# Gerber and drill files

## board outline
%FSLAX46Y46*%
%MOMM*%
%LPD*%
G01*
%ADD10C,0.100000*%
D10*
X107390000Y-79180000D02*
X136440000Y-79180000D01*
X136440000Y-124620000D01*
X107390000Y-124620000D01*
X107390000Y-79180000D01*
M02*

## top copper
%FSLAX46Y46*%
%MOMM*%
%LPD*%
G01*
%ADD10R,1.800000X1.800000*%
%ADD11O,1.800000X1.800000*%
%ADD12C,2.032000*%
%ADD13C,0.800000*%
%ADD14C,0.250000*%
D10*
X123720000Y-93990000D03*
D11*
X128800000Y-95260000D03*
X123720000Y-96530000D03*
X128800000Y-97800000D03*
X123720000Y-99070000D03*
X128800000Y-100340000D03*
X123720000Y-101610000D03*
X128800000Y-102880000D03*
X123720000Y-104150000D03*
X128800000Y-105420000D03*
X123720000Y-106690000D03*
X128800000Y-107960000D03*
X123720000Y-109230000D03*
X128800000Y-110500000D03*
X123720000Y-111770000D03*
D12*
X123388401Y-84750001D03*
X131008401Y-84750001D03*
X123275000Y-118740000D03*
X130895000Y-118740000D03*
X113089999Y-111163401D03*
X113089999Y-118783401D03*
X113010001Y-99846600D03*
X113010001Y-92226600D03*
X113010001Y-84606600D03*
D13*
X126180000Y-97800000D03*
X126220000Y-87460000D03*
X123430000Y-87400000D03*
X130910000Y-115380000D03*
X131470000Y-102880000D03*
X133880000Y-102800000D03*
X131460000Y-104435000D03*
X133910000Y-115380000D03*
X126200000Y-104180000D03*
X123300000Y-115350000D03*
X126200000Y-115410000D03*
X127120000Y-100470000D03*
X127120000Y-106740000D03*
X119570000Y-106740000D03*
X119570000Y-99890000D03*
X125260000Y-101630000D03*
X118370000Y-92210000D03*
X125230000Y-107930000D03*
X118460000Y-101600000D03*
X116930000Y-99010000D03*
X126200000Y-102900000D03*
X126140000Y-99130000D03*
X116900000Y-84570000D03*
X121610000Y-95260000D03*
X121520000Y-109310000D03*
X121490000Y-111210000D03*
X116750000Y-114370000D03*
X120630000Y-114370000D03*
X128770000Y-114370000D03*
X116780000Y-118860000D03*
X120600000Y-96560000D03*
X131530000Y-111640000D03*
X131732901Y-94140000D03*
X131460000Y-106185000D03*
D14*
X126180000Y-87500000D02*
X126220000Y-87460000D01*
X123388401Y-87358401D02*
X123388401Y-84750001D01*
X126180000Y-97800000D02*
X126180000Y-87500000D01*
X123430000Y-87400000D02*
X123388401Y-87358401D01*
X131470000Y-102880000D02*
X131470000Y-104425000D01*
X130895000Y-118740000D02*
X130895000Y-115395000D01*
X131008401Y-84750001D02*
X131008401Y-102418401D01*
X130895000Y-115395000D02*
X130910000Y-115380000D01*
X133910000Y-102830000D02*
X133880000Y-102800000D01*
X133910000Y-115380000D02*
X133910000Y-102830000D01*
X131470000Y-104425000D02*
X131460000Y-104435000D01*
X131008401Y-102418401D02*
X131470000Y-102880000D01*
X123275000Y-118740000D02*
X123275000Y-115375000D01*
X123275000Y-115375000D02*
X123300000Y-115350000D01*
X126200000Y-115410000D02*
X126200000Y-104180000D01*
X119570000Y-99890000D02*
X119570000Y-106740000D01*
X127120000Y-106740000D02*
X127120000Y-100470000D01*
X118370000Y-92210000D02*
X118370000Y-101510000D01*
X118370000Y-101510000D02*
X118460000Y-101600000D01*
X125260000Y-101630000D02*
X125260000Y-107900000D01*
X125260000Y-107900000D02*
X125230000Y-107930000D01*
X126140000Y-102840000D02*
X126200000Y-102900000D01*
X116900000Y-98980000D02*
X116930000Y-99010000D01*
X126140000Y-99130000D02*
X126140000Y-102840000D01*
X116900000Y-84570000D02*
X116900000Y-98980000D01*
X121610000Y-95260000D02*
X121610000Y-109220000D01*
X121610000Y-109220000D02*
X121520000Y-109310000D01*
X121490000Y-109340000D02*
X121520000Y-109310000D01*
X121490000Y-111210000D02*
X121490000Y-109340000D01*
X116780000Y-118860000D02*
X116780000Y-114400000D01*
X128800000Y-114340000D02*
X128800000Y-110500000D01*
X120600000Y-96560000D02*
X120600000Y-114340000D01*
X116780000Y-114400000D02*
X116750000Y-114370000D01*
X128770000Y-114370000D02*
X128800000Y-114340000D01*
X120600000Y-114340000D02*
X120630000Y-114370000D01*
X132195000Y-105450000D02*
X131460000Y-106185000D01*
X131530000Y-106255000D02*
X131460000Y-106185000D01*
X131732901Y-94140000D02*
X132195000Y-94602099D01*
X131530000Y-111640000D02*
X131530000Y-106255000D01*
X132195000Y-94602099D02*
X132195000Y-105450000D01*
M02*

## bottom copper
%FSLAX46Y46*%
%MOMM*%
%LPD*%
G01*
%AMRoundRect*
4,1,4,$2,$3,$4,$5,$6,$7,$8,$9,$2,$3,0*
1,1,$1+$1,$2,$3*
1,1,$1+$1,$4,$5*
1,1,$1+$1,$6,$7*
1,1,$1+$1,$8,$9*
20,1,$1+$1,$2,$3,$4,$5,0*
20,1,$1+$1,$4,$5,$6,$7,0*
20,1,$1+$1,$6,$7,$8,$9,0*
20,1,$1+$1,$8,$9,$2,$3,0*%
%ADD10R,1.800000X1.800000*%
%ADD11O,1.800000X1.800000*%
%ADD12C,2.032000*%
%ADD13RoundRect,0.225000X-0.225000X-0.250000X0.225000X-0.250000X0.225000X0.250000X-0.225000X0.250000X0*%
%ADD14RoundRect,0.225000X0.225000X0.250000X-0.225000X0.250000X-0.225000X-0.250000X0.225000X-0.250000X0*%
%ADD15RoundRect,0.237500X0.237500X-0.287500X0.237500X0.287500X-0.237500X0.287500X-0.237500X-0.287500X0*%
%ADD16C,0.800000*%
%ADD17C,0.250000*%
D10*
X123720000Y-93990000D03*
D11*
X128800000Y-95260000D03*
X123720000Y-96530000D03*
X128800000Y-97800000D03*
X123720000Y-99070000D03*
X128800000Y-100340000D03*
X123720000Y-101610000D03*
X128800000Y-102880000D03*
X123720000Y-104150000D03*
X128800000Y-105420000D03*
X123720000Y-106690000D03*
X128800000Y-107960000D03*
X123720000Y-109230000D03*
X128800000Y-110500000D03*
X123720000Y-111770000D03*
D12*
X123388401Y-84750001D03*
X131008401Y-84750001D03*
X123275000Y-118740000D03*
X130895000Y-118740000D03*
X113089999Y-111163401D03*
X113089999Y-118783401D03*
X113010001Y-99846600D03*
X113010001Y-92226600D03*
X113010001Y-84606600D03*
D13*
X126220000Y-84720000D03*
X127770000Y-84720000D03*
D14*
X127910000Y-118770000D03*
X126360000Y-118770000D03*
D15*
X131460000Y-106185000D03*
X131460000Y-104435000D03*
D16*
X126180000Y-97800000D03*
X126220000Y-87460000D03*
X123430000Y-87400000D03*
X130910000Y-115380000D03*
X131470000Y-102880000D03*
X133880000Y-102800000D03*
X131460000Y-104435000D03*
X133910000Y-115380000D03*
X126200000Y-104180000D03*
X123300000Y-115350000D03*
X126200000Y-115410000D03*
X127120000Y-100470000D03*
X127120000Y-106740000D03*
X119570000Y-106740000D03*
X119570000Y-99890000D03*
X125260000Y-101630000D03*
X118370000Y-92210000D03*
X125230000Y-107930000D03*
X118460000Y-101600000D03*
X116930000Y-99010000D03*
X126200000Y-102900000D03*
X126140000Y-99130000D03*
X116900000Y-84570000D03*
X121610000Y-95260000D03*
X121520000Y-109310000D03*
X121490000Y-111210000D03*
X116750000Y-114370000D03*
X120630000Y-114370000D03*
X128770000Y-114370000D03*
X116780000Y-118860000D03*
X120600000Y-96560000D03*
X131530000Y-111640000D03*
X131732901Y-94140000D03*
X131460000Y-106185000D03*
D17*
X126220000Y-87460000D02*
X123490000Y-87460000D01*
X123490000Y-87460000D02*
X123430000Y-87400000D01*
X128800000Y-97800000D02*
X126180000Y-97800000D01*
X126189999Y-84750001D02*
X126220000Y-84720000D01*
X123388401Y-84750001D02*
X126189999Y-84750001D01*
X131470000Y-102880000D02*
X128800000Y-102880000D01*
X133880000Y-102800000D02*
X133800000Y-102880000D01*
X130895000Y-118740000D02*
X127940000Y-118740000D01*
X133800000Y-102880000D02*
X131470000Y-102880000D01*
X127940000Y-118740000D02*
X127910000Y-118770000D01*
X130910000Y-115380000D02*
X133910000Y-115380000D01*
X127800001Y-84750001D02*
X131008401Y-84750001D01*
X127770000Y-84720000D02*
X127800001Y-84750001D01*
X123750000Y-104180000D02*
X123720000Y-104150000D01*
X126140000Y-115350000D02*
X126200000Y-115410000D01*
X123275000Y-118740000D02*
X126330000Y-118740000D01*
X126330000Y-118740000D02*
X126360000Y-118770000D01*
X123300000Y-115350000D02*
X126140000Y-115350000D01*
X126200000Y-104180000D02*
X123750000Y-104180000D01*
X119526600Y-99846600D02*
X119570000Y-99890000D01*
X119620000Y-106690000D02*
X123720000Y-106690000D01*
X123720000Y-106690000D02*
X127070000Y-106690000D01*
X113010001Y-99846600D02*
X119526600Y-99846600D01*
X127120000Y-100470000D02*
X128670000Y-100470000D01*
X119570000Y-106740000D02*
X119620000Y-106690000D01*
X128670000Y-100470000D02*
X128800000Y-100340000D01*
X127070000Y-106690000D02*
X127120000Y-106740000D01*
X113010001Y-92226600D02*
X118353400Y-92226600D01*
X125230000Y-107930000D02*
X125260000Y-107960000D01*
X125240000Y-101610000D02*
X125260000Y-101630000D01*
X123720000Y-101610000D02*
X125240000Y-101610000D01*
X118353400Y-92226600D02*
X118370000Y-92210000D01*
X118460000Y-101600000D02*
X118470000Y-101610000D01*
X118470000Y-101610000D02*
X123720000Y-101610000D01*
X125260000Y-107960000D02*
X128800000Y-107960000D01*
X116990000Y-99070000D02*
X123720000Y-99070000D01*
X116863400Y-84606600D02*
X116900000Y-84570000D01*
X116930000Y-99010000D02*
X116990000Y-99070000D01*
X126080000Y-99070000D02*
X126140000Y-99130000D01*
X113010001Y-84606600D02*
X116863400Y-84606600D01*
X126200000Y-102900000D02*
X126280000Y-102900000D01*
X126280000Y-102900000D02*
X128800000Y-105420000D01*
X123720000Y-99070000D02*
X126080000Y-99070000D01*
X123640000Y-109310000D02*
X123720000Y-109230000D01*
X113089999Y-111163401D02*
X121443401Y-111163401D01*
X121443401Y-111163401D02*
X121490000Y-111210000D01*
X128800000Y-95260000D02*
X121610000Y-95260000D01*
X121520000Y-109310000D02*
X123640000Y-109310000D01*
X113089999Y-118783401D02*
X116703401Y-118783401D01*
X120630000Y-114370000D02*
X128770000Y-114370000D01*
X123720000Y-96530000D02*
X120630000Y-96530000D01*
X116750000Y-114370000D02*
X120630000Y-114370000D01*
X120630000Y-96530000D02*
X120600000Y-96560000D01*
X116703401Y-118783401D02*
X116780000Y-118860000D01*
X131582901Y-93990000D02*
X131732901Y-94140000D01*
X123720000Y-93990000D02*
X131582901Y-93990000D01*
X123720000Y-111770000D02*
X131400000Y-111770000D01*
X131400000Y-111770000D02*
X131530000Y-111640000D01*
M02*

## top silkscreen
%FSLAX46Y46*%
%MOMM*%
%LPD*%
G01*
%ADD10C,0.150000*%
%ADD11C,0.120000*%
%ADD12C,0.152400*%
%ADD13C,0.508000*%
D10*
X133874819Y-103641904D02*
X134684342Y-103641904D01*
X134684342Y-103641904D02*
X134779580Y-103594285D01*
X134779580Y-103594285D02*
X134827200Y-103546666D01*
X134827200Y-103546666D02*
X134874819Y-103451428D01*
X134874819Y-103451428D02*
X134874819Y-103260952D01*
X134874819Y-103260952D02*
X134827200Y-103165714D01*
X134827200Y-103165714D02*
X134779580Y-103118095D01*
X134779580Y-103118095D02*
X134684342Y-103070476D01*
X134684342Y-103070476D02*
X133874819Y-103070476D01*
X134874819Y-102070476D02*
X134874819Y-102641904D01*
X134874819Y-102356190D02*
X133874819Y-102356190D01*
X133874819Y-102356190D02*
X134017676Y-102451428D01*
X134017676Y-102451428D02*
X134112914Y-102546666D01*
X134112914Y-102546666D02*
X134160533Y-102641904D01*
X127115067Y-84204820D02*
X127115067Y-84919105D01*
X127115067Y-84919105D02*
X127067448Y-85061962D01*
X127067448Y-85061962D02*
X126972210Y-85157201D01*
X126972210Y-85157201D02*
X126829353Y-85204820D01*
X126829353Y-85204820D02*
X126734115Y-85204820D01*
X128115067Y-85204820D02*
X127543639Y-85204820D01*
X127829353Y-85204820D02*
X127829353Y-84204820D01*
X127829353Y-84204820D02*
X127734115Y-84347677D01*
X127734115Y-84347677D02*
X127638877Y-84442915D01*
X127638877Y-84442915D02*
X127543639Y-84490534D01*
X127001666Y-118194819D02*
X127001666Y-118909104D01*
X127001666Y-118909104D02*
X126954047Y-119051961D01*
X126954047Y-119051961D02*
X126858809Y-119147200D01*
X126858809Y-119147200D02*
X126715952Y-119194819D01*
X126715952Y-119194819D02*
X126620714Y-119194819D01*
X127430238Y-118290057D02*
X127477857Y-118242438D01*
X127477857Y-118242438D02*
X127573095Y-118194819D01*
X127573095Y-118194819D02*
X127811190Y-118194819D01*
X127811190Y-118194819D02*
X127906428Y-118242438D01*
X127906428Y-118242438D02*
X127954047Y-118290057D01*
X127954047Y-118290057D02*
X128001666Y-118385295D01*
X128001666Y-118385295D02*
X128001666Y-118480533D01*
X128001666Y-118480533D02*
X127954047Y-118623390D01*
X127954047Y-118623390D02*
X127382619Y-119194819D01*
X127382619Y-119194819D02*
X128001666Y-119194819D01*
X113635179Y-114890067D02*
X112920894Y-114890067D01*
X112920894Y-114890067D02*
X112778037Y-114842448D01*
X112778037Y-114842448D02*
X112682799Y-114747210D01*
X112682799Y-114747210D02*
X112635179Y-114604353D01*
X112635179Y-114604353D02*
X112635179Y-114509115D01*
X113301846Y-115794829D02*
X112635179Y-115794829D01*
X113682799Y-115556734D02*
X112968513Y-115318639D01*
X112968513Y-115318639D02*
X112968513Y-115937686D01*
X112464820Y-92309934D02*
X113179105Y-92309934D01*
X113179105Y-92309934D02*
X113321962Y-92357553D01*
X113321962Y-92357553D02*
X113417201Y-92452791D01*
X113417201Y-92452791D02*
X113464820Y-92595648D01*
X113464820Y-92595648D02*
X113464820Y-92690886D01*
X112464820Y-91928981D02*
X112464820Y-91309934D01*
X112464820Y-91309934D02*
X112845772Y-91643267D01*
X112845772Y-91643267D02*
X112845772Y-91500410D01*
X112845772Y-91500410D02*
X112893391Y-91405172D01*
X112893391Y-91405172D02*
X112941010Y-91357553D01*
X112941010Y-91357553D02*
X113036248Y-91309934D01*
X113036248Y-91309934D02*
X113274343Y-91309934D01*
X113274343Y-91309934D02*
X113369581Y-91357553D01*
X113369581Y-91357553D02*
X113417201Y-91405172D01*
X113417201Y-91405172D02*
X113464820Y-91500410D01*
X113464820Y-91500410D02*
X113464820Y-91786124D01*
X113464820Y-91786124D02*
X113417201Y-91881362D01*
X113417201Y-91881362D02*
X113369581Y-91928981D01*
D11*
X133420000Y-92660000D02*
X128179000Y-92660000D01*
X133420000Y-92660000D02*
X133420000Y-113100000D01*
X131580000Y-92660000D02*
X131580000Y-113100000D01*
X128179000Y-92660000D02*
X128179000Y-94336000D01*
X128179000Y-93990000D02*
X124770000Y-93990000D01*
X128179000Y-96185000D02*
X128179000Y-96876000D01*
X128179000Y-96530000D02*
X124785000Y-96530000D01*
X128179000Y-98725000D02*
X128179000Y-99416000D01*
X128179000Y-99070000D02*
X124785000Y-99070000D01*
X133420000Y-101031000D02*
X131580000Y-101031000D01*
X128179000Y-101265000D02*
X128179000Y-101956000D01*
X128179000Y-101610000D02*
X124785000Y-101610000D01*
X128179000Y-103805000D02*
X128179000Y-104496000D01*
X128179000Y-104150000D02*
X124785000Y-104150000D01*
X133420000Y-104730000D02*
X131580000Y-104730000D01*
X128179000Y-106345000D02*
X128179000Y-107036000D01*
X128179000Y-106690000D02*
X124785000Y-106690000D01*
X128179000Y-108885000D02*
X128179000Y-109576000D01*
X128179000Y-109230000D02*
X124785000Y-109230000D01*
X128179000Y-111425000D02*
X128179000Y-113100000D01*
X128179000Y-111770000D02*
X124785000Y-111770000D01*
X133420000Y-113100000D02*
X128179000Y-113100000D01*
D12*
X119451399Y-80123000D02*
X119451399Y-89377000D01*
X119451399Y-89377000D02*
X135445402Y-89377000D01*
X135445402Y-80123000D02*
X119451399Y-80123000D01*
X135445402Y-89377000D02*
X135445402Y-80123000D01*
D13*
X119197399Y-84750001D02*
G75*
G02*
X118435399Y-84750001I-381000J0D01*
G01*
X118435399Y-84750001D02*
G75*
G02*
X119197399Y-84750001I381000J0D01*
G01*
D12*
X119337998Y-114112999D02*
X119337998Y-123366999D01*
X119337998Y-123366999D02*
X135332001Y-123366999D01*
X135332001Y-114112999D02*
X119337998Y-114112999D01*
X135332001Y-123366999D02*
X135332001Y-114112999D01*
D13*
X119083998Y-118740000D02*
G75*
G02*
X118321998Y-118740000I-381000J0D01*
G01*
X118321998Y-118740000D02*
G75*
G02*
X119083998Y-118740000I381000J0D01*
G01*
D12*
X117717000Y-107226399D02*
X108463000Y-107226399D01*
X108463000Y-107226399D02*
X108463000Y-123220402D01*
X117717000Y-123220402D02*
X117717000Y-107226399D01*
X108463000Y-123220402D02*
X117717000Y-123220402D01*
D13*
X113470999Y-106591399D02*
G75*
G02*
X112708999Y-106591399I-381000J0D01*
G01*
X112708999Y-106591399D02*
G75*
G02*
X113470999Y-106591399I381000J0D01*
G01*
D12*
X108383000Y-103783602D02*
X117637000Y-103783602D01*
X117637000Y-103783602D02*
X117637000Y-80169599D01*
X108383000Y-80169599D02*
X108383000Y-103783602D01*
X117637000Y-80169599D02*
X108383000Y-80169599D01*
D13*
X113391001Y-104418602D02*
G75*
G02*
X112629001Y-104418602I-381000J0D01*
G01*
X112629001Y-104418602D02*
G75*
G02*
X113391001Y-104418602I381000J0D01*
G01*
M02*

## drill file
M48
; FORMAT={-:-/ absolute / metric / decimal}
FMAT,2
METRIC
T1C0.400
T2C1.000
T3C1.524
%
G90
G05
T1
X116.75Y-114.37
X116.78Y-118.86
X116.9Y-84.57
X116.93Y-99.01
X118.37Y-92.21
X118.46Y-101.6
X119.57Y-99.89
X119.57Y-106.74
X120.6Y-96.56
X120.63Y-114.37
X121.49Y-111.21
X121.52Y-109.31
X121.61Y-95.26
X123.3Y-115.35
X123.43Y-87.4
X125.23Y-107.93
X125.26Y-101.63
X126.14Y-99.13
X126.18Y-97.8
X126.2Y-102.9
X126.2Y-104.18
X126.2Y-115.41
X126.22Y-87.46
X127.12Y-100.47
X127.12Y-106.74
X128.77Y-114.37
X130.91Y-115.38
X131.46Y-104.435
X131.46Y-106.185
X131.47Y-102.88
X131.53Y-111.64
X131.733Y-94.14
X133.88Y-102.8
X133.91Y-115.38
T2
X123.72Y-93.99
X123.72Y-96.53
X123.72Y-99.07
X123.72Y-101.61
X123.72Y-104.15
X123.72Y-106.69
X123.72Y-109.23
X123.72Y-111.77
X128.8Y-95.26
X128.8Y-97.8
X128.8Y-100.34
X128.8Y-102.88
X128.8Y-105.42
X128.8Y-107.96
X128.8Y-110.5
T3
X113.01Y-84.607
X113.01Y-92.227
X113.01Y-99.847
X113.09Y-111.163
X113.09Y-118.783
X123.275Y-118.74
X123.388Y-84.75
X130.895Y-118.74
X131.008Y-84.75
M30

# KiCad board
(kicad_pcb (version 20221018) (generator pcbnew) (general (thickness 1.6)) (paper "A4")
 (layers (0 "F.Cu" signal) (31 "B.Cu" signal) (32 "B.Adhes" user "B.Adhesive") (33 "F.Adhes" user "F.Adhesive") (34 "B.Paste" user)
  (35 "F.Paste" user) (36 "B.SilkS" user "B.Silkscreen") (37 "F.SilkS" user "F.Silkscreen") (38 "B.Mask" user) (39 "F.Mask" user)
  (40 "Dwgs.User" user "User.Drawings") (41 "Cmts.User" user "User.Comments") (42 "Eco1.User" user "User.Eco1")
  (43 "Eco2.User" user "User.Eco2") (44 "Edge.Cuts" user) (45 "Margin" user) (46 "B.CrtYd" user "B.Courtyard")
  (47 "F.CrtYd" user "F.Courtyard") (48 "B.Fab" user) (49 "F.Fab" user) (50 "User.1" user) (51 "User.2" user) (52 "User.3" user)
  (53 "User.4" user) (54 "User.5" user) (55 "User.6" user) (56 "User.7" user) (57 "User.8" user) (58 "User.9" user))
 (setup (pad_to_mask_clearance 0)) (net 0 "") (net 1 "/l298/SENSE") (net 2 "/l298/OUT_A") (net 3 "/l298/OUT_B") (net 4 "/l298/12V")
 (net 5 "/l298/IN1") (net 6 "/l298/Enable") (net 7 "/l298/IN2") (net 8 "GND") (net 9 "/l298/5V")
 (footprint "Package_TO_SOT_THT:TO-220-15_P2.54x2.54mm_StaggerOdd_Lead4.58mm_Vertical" (layer "F.Cu") (at 123.72 93.99 -90)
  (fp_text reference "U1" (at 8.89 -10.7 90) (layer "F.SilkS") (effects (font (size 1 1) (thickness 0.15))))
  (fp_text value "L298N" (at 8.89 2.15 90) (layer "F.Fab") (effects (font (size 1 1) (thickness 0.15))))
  (fp_line (start -1.33 -9.7) (end -1.33 -4.459) (stroke (width 0.12) (type solid)) (layer "F.SilkS"))
  (fp_line (start -1.33 -9.7) (end 19.11 -9.7) (stroke (width 0.12) (type solid)) (layer "F.SilkS"))
  (fp_line (start -1.33 -7.86) (end 19.11 -7.86) (stroke (width 0.12) (type solid)) (layer "F.SilkS"))
  (fp_line (start -1.33 -4.459) (end 0.346 -4.459) (stroke (width 0.12) (type solid)) (layer "F.SilkS"))
  (fp_line (start 0 -4.459) (end 0 -1.05) (stroke (width 0.12) (type solid)) (layer "F.SilkS"))
  (fp_line (start 2.195 -4.459) (end 2.886 -4.459) (stroke (width 0.12) (type solid)) (layer "F.SilkS"))
  (fp_line (start 2.54 -4.459) (end 2.54 -1.065) (stroke (width 0.12) (type solid)) (layer "F.SilkS"))
  (fp_line (start 4.735 -4.459) (end 5.426 -4.459) (stroke (width 0.12) (type solid)) (layer "F.SilkS"))
  (fp_line (start 5.08 -4.459) (end 5.08 -1.065) (stroke (width 0.12) (type solid)) (layer "F.SilkS"))
  (fp_line (start 7.041 -9.7) (end 7.041 -7.86) (stroke (width 0.12) (type solid)) (layer "F.SilkS"))
  (fp_line (start 7.275 -4.459) (end 7.966 -4.459) (stroke (width 0.12) (type solid)) (layer "F.SilkS"))
  (fp_line (start 7.62 -4.459) (end 7.62 -1.065) (stroke (width 0.12) (type solid)) (layer "F.SilkS"))
  (fp_line (start 9.815 -4.459) (end 10.506 -4.459) (stroke (width 0.12) (type solid)) (layer "F.SilkS"))
  (fp_line (start 10.16 -4.459) (end 10.16 -1.065) (stroke (width 0.12) (type solid)) (layer "F.SilkS"))
  (fp_line (start 10.74 -9.7) (end 10.74 -7.86) (stroke (width 0.12) (type solid)) (layer "F.SilkS"))
  (fp_line (start 12.355 -4.459) (end 13.046 -4.459) (stroke (width 0.12) (type solid)) (layer "F.SilkS"))
  (fp_line (start 12.7 -4.459) (end 12.7 -1.065) (stroke (width 0.12) (type solid)) (layer "F.SilkS"))
  (fp_line (start 14.895 -4.459) (end 15.586 -4.459) (stroke (width 0.12) (type solid)) (layer "F.SilkS"))
  (fp_line (start 15.24 -4.459) (end 15.24 -1.065) (stroke (width 0.12) (type solid)) (layer "F.SilkS"))
  (fp_line (start 17.435 -4.459) (end 19.11 -4.459) (stroke (width 0.12) (type solid)) (layer "F.SilkS"))
  (fp_line (start 17.78 -4.459) (end 17.78 -1.065) (stroke (width 0.12) (type solid)) (layer "F.SilkS"))
  (fp_line (start 19.11 -9.7) (end 19.11 -4.459) (stroke (width 0.12) (type solid)) (layer "F.SilkS"))
  (pad "1" thru_hole rect (at 0 0 270) (size 1.8 1.8) (drill 1) (layers "*.Cu" "*.Mask") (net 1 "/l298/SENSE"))
  (pad "2" thru_hole oval (at 1.27 -5.08 270) (size 1.8 1.8) (drill 1) (layers "*.Cu" "*.Mask") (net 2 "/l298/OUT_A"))
  (pad "3" thru_hole oval (at 2.54 0 270) (size 1.8 1.8) (drill 1) (layers "*.Cu" "*.Mask") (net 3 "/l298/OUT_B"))
  (pad "4" thru_hole oval (at 3.81 -5.08 270) (size 1.8 1.8) (drill 1) (layers "*.Cu" "*.Mask") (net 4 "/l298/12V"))
  (pad "5" thru_hole oval (at 5.08 0 270) (size 1.8 1.8) (drill 1) (layers "*.Cu" "*.Mask") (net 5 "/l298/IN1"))
  (pad "6" thru_hole oval (at 6.35 -5.08 270) (size 1.8 1.8) (drill 1) (layers "*.Cu" "*.Mask") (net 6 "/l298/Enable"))
  (pad "7" thru_hole oval (at 7.62 0 270) (size 1.8 1.8) (drill 1) (layers "*.Cu" "*.Mask") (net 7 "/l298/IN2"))
  (pad "8" thru_hole oval (at 8.89 -5.08 270) (size 1.8 1.8) (drill 1) (layers "*.Cu" "*.Mask") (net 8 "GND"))
  (pad "9" thru_hole oval (at 10.16 0 270) (size 1.8 1.8) (drill 1) (layers "*.Cu" "*.Mask") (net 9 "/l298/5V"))
  (pad "10" thru_hole oval (at 11.43 -5.08 270) (size 1.8 1.8) (drill 1) (layers "*.Cu" "*.Mask") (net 5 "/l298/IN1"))
  (pad "11" thru_hole oval (at 12.7 0 270) (size 1.8 1.8) (drill 1) (layers "*.Cu" "*.Mask") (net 6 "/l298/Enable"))
  (pad "12" thru_hole oval (at 13.97 -5.08 270) (size 1.8 1.8) (drill 1) (layers "*.Cu" "*.Mask") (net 7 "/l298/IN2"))
  (pad "13" thru_hole oval (at 15.24 0 270) (size 1.8 1.8) (drill 1) (layers "*.Cu" "*.Mask") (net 2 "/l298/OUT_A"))
  (pad "14" thru_hole oval (at 16.51 -5.08 270) (size 1.8 1.8) (drill 1) (layers "*.Cu" "*.Mask") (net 3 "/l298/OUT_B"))
  (pad "15" thru_hole oval (at 17.78 0 270) (size 1.8 1.8) (drill 1) (layers "*.Cu" "*.Mask") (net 1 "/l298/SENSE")))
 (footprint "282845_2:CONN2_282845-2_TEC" (layer "F.Cu") (at 123.388401 84.750001)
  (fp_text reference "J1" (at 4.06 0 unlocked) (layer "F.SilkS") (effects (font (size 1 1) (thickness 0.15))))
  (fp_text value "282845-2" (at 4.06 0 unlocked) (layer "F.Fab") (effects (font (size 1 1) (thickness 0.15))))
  (fp_line (start -3.937002 -4.627001) (end -3.937002 4.626999) (stroke (width 0.1524) (type solid)) (layer "F.SilkS"))
  (fp_line (start -3.937002 4.626999) (end 12.057001 4.626999) (stroke (width 0.1524) (type solid)) (layer "F.SilkS"))
  (fp_line (start 12.057001 -4.627001) (end -3.937002 -4.627001) (stroke (width 0.1524) (type solid)) (layer "F.SilkS"))
  (fp_line (start 12.057001 4.626999) (end 12.057001 -4.627001) (stroke (width 0.1524) (type solid)) (layer "F.SilkS"))
  (fp_circle (center -4.572002 0) (end -4.191002 0) (stroke (width 0.508) (type solid)) (fill none) (layer "F.SilkS"))
  (pad "1" thru_hole circle (at 0 0) (size 2.032 2.032) (drill 1.524) (layers "*.Cu" "*.Mask") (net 4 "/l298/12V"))
  (pad "2" thru_hole circle (at 7.62 0) (size 2.032 2.032) (drill 1.524) (layers "*.Cu" "*.Mask") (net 8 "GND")))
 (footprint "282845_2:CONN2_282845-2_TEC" (layer "F.Cu") (at 123.275 118.74)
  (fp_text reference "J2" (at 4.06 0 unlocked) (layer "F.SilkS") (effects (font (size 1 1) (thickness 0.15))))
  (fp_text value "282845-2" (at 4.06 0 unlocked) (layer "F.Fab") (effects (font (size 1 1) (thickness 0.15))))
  (fp_line (start -3.937002 -4.627001) (end -3.937002 4.626999) (stroke (width 0.1524) (type solid)) (layer "F.SilkS"))
  (fp_line (start -3.937002 4.626999) (end 12.057001 4.626999) (stroke (width 0.1524) (type solid)) (layer "F.SilkS"))
  (fp_line (start 12.057001 -4.627001) (end -3.937002 -4.627001) (stroke (width 0.1524) (type solid)) (layer "F.SilkS"))
  (fp_line (start 12.057001 4.626999) (end 12.057001 -4.627001) (stroke (width 0.1524) (type solid)) (layer "F.SilkS"))
  (fp_circle (center -4.572002 0) (end -4.191002 0) (stroke (width 0.508) (type solid)) (fill none) (layer "F.SilkS"))
  (pad "1" thru_hole circle (at 0 0) (size 2.032 2.032) (drill 1.524) (layers "*.Cu" "*.Mask") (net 9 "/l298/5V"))
  (pad "2" thru_hole circle (at 7.62 0) (size 2.032 2.032) (drill 1.524) (layers "*.Cu" "*.Mask") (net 8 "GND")))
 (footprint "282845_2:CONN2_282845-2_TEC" (layer "F.Cu") (at 113.089999 111.163401 -90)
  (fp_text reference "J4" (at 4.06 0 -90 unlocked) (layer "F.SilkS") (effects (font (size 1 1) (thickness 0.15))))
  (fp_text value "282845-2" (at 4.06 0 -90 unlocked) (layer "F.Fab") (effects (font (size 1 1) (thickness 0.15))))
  (fp_line (start -3.937002 -4.627001) (end -3.937002 4.626999) (stroke (width 0.1524) (type solid)) (layer "F.SilkS"))
  (fp_line (start -3.937002 4.626999) (end 12.057001 4.626999) (stroke (width 0.1524) (type solid)) (layer "F.SilkS"))
  (fp_line (start 12.057001 -4.627001) (end -3.937002 -4.627001) (stroke (width 0.1524) (type solid)) (layer "F.SilkS"))
  (fp_line (start 12.057001 4.626999) (end 12.057001 -4.627001) (stroke (width 0.1524) (type solid)) (layer "F.SilkS"))
  (fp_circle (center -4.572002 0) (end -4.191002 0) (stroke (width 0.508) (type solid)) (fill none) (layer "F.SilkS"))
  (pad "1" thru_hole circle (at 0 0 270) (size 2.032 2.032) (drill 1.524) (layers "*.Cu" "*.Mask") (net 2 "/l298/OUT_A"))
  (pad "2" thru_hole circle (at 7.62 0 270) (size 2.032 2.032) (drill 1.524) (layers "*.Cu" "*.Mask") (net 3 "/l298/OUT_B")))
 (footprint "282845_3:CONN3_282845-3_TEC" (layer "F.Cu") (at 113.010001 99.8466 90)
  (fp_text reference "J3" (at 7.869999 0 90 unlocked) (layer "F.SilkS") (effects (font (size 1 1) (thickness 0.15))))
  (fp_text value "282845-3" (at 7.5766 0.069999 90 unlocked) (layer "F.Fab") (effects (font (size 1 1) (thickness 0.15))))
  (fp_line (start -3.937002 -4.627001) (end -3.937002 4.626999) (stroke (width 0.1524) (type solid)) (layer "F.SilkS"))
  (fp_line (start -3.937002 4.626999) (end 19.677001 4.626999) (stroke (width 0.1524) (type solid)) (layer "F.SilkS"))
  (fp_line (start 19.677001 -4.627001) (end -3.937002 -4.627001) (stroke (width 0.1524) (type solid)) (layer "F.SilkS"))
  (fp_line (start 19.677001 4.626999) (end 19.677001 -4.627001) (stroke (width 0.1524) (type solid)) (layer "F.SilkS"))
  (fp_circle (center -4.572002 0) (end -4.191002 0) (stroke (width 0.508) (type solid)) (fill none) (layer "F.SilkS"))
  (pad "1" thru_hole circle (at 0 0 90) (size 2.032 2.032) (drill 1.524) (layers "*.Cu" "*.Mask") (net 6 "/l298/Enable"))
  (pad "2" thru_hole circle (at 7.62 0 90) (size 2.032 2.032) (drill 1.524) (layers "*.Cu" "*.Mask") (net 7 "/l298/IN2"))
  (pad "3" thru_hole circle (at 15.24 0 90) (size 2.032 2.032) (drill 1.524) (layers "*.Cu" "*.Mask") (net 5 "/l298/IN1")))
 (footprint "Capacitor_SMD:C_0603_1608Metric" (layer "B.Cu") (at 126.995 84.72)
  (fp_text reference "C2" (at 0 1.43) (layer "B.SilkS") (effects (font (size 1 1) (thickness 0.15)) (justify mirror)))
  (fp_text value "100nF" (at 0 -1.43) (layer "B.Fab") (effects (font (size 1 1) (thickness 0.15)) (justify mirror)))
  (pad "1" smd roundrect (at -0.775 0) (size 0.9 0.95) (layers "B.Cu" "B.Paste" "B.Mask") (roundrect_rratio 0.25) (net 4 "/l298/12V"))
  (pad "2" smd roundrect (at 0.775 0) (size 0.9 0.95) (layers "B.Cu" "B.Paste" "B.Mask") (roundrect_rratio 0.25) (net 8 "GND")))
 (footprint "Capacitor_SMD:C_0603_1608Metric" (layer "B.Cu") (at 127.135 118.77 180)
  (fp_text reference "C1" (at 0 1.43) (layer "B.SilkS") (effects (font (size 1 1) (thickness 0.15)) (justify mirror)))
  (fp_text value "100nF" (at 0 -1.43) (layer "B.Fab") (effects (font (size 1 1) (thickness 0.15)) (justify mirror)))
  (pad "1" smd roundrect (at -0.775 0 180) (size 0.9 0.95) (layers "B.Cu" "B.Paste" "B.Mask") (roundrect_rratio 0.25) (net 8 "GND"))
  (pad "2" smd roundrect (at 0.775 0 180) (size 0.9 0.95) (layers "B.Cu" "B.Paste" "B.Mask") (roundrect_rratio 0.25) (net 9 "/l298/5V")))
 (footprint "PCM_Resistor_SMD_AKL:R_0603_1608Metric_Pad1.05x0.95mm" (layer "B.Cu") (at 131.46 105.31 90)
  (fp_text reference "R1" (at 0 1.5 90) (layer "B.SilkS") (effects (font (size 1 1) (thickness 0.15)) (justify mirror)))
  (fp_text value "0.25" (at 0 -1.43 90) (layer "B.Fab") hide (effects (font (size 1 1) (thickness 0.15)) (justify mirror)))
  (pad "1" smd roundrect (at -0.875 0 90) (size 1.05 0.95) (layers "B.Cu" "B.Paste" "B.Mask") (roundrect_rratio 0.25) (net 1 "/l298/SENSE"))
  (pad "2" smd roundrect (at 0.875 0 90) (size 1.05 0.95) (layers "B.Cu" "B.Paste" "B.Mask") (roundrect_rratio 0.25) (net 8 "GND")))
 (gr_rect (start 107.39 79.18) (end 136.44 124.62) (stroke (width 0.1) (type default)) (fill none) (layer "Edge.Cuts"))
 (segment (start 126.18 87.5) (end 126.22 87.46) (width 0.25) (layer "F.Cu") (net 4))
 (segment (start 123.388401 87.358401) (end 123.388401 84.750001) (width 0.25) (layer "F.Cu") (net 4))
 (segment (start 126.18 97.8) (end 126.18 87.5) (width 0.25) (layer "F.Cu") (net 4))
 (segment (start 123.43 87.4) (end 123.388401 87.358401) (width 0.25) (layer "F.Cu") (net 4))
 (via (at 126.18 97.8) (size 0.8) (drill 0.4) (layers "F.Cu" "B.Cu") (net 4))
 (via (at 126.22 87.46) (size 0.8) (drill 0.4) (layers "F.Cu" "B.Cu") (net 4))
 (via (at 123.43 87.4) (size 0.8) (drill 0.4) (layers "F.Cu" "B.Cu") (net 4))
 (segment (start 126.22 87.46) (end 123.49 87.46) (width 0.25) (layer "B.Cu") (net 4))
 (segment (start 123.49 87.46) (end 123.43 87.4) (width 0.25) (layer "B.Cu") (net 4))
 (segment (start 128.8 97.8) (end 126.18 97.8) (width 0.25) (layer "B.Cu") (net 4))
 (segment (start 126.189999 84.750001) (end 126.22 84.72) (width 0.25) (layer "B.Cu") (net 4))
 (segment (start 123.388401 84.750001) (end 126.189999 84.750001) (width 0.25) (layer "B.Cu") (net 4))
 (segment (start 131.47 102.88) (end 131.47 104.425) (width 0.25) (layer "F.Cu") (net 8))
 (segment (start 130.895 118.74) (end 130.895 115.395) (width 0.25) (layer "F.Cu") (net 8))
 (segment (start 131.008401 84.750001) (end 131.008401 102.418401) (width 0.25) (layer "F.Cu") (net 8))
 (segment (start 130.895 115.395) (end 130.91 115.38) (width 0.25) (layer "F.Cu") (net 8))
 (segment (start 133.91 102.83) (end 133.88 102.8) (width 0.25) (layer "F.Cu") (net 8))
 (segment (start 133.91 115.38) (end 133.91 102.83) (width 0.25) (layer "F.Cu") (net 8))
 (segment (start 131.47 104.425) (end 131.46 104.435) (width 0.25) (layer "F.Cu") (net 8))
 (segment (start 131.008401 102.418401) (end 131.47 102.88) (width 0.25) (layer "F.Cu") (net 8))
 (via (at 130.91 115.38) (size 0.8) (drill 0.4) (layers "F.Cu" "B.Cu") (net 8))
 (via (at 131.47 102.88) (size 0.8) (drill 0.4) (layers "F.Cu" "B.Cu") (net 8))
 (via (at 133.88 102.8) (size 0.8) (drill 0.4) (layers "F.Cu" "B.Cu") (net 8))
 (via (at 131.46 104.435) (size 0.8) (drill 0.4) (layers "F.Cu" "B.Cu") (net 8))
 (via (at 133.91 115.38) (size 0.8) (drill 0.4) (layers "F.Cu" "B.Cu") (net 8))
 (segment (start 131.47 102.88) (end 128.8 102.88) (width 0.25) (layer "B.Cu") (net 8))
 (segment (start 133.88 102.8) (end 133.8 102.88) (width 0.25) (layer "B.Cu") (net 8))
 (segment (start 130.895 118.74) (end 127.94 118.74) (width 0.25) (layer "B.Cu") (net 8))
 (segment (start 133.8 102.88) (end 131.47 102.88) (width 0.25) (layer "B.Cu") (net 8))
 (segment (start 127.94 118.74) (end 127.91 118.77) (width 0.25) (layer "B.Cu") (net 8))
 (segment (start 130.91 115.38) (end 133.91 115.38) (width 0.25) (layer "B.Cu") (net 8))
 (segment (start 127.800001 84.750001) (end 131.008401 84.750001) (width 0.25) (layer "B.Cu") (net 8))
 (segment (start 127.77 84.72) (end 127.800001 84.750001) (width 0.25) (layer "B.Cu") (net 8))
 (segment (start 123.275 118.74) (end 123.275 115.375) (width 0.25) (layer "F.Cu") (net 9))
 (segment (start 123.275 115.375) (end 123.3 115.35) (width 0.25) (layer "F.Cu") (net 9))
 (segment (start 126.2 115.41) (end 126.2 104.18) (width 0.25) (layer "F.Cu") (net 9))
 (via (at 126.2 104.18) (size 0.8) (drill 0.4) (layers "F.Cu" "B.Cu") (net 9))
 (via (at 123.3 115.35) (size 0.8) (drill 0.4) (layers "F.Cu" "B.Cu") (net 9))
 (via (at 126.2 115.41) (size 0.8) (drill 0.4) (layers "F.Cu" "B.Cu") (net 9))
 (segment (start 123.75 104.18) (end 123.72 104.15) (width 0.25) (layer "B.Cu") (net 9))
 (segment (start 126.14 115.35) (end 126.2 115.41) (width 0.25) (layer "B.Cu") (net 9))
 (segment (start 123.275 118.74) (end 126.33 118.74) (width 0.25) (layer "B.Cu") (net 9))
 (segment (start 126.33 118.74) (end 126.36 118.77) (width 0.25) (layer "B.Cu") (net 9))
 (segment (start 123.3 115.35) (end 126.14 115.35) (width 0.25) (layer "B.Cu") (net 9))
 (segment (start 126.2 104.18) (end 123.75 104.18) (width 0.25) (layer "B.Cu") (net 9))
 (segment (start 119.57 99.89) (end 119.57 106.74) (width 0.25) (layer "F.Cu") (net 6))
 (segment (start 127.12 106.74) (end 127.12 100.47) (width 0.25) (layer "F.Cu") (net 6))
 (via (at 127.12 100.47) (size 0.8) (drill 0.4) (layers "F.Cu" "B.Cu") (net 6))
 (via (at 127.12 106.74) (size 0.8) (drill 0.4) (layers "F.Cu" "B.Cu") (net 6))
 (via (at 119.57 106.74) (size 0.8) (drill 0.4) (layers "F.Cu" "B.Cu") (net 6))
 (via (at 119.57 99.89) (size 0.8) (drill 0.4) (layers "F.Cu" "B.Cu") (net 6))
 (segment (start 119.5266 99.8466) (end 119.57 99.89) (width 0.25) (layer "B.Cu") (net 6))
 (segment (start 119.62 106.69) (end 123.72 106.69) (width 0.25) (layer "B.Cu") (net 6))
 (segment (start 123.72 106.69) (end 127.07 106.69) (width 0.25) (layer "B.Cu") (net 6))
 (segment (start 113.010001 99.8466) (end 119.5266 99.8466) (width 0.25) (layer "B.Cu") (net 6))
 (segment (start 127.12 100.47) (end 128.67 100.47) (width 0.25) (layer "B.Cu") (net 6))
 (segment (start 119.57 106.74) (end 119.62 106.69) (width 0.25) (layer "B.Cu") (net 6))
 (segment (start 128.67 100.47) (end 128.8 100.34) (width 0.25) (layer "B.Cu") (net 6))
 (segment (start 127.07 106.69) (end 127.12 106.74) (width 0.25) (layer "B.Cu") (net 6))
 (segment (start 118.37 92.21) (end 118.37 101.51) (width 0.25) (layer "F.Cu") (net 7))
 (segment (start 118.37 101.51) (end 118.46 101.6) (width 0.25) (layer "F.Cu") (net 7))
 (segment (start 125.26 101.63) (end 125.26 107.9) (width 0.25) (layer "F.Cu") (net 7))
 (segment (start 125.26 107.9) (end 125.23 107.93) (width 0.25) (layer "F.Cu") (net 7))
 (via (at 125.26 101.63) (size 0.8) (drill 0.4) (layers "F.Cu" "B.Cu") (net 7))
 (via (at 118.37 92.21) (size 0.8) (drill 0.4) (layers "F.Cu" "B.Cu") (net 7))
 (via (at 125.23 107.93) (size 0.8) (drill 0.4) (layers "F.Cu" "B.Cu") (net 7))
 (via (at 118.46 101.6) (size 0.8) (drill 0.4) (layers "F.Cu" "B.Cu") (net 7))
 (segment (start 113.010001 92.2266) (end 118.3534 92.2266) (width 0.25) (layer "B.Cu") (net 7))
 (segment (start 125.23 107.93) (end 125.26 107.96) (width 0.25) (layer "B.Cu") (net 7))
 (segment (start 125.24 101.61) (end 125.26 101.63) (width 0.25) (layer "B.Cu") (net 7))
 (segment (start 123.72 101.61) (end 125.24 101.61) (width 0.25) (layer "B.Cu") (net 7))
 (segment (start 118.3534 92.2266) (end 118.37 92.21) (width 0.25) (layer "B.Cu") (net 7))
 (segment (start 118.46 101.6) (end 118.47 101.61) (width 0.25) (layer "B.Cu") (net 7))
 (segment (start 118.47 101.61) (end 123.72 101.61) (width 0.25) (layer "B.Cu") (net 7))
 (segment (start 125.26 107.96) (end 128.8 107.96) (width 0.25) (layer "B.Cu") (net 7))
 (segment (start 126.14 102.84) (end 126.2 102.9) (width 0.25) (layer "F.Cu") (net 5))
 (segment (start 116.9 98.98) (end 116.93 99.01) (width 0.25) (layer "F.Cu") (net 5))
 (segment (start 126.14 99.13) (end 126.14 102.84) (width 0.25) (layer "F.Cu") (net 5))
 (segment (start 116.9 84.57) (end 116.9 98.98) (width 0.25) (layer "F.Cu") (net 5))
 (via (at 116.93 99.01) (size 0.8) (drill 0.4) (layers "F.Cu" "B.Cu") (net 5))
 (via (at 126.2 102.9) (size 0.8) (drill 0.4) (layers "F.Cu" "B.Cu") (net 5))
 (via (at 126.14 99.13) (size 0.8) (drill 0.4) (layers "F.Cu" "B.Cu") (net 5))
 (via (at 116.9 84.57) (size 0.8) (drill 0.4) (layers "F.Cu" "B.Cu") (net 5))
 (segment (start 116.99 99.07) (end 123.72 99.07) (width 0.25) (layer "B.Cu") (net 5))
 (segment (start 116.8634 84.6066) (end 116.9 84.57) (width 0.25) (layer "B.Cu") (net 5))
 (segment (start 116.93 99.01) (end 116.99 99.07) (width 0.25) (layer "B.Cu") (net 5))
 (segment (start 126.08 99.07) (end 126.14 99.13) (width 0.25) (layer "B.Cu") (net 5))
 (segment (start 113.010001 84.6066) (end 116.8634 84.6066) (width 0.25) (layer "B.Cu") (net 5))
 (segment (start 126.2 102.9) (end 126.28 102.9) (width 0.25) (layer "B.Cu") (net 5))
 (segment (start 126.28 102.9) (end 128.8 105.42) (width 0.25) (layer "B.Cu") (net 5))
 (segment (start 123.72 99.07) (end 126.08 99.07) (width 0.25) (layer "B.Cu") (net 5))
 (segment (start 121.61 95.26) (end 121.61 109.22) (width 0.25) (layer "F.Cu") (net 2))
 (segment (start 121.61 109.22) (end 121.52 109.31) (width 0.25) (layer "F.Cu") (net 2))
 (segment (start 121.49 109.34) (end 121.52 109.31) (width 0.25) (layer "F.Cu") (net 2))
 (segment (start 121.49 111.21) (end 121.49 109.34) (width 0.25) (layer "F.Cu") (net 2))
 (via (at 121.61 95.26) (size 0.8) (drill 0.4) (layers "F.Cu" "B.Cu") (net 2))
 (via (at 121.52 109.31) (size 0.8) (drill 0.4) (layers "F.Cu" "B.Cu") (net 2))
 (via (at 121.49 111.21) (size 0.8) (drill 0.4) (layers "F.Cu" "B.Cu") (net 2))
 (segment (start 123.64 109.31) (end 123.72 109.23) (width 0.25) (layer "B.Cu") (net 2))
 (segment (start 113.089999 111.163401) (end 121.443401 111.163401) (width 0.25) (layer "B.Cu") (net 2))
 (segment (start 121.443401 111.163401) (end 121.49 111.21) (width 0.25) (layer "B.Cu") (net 2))
 (segment (start 128.8 95.26) (end 121.61 95.26) (width 0.25) (layer "B.Cu") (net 2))
 (segment (start 121.52 109.31) (end 123.64 109.31) (width 0.25) (layer "B.Cu") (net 2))
 (segment (start 116.78 118.86) (end 116.78 114.4) (width 0.25) (layer "F.Cu") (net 3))
 (segment (start 128.8 114.34) (end 128.8 110.5) (width 0.25) (layer "F.Cu") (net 3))
 (segment (start 120.6 96.56) (end 120.6 114.34) (width 0.25) (layer "F.Cu") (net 3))
 (segment (start 116.78 114.4) (end 116.75 114.37) (width 0.25) (layer "F.Cu") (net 3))
 (segment (start 128.77 114.37) (end 128.8 114.34) (width 0.25) (layer "F.Cu") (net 3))
 (segment (start 120.6 114.34) (end 120.63 114.37) (width 0.25) (layer "F.Cu") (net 3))
 (via (at 116.75 114.37) (size 0.8) (drill 0.4) (layers "F.Cu" "B.Cu") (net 3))
 (via (at 120.63 114.37) (size 0.8) (drill 0.4) (layers "F.Cu" "B.Cu") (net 3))
 (via (at 128.77 114.37) (size 0.8) (drill 0.4) (layers "F.Cu" "B.Cu") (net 3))
 (via (at 116.78 118.86) (size 0.8) (drill 0.4) (layers "F.Cu" "B.Cu") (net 3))
 (via (at 120.6 96.56) (size 0.8) (drill 0.4) (layers "F.Cu" "B.Cu") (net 3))
 (segment (start 113.089999 118.783401) (end 116.703401 118.783401) (width 0.25) (layer "B.Cu") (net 3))
 (segment (start 120.63 114.37) (end 128.77 114.37) (width 0.25) (layer "B.Cu") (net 3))
 (segment (start 123.72 96.53) (end 120.63 96.53) (width 0.25) (layer "B.Cu") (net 3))
 (segment (start 116.75 114.37) (end 120.63 114.37) (width 0.25) (layer "B.Cu") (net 3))
 (segment (start 120.63 96.53) (end 120.6 96.56) (width 0.25) (layer "B.Cu") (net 3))
 (segment (start 116.703401 118.783401) (end 116.78 118.86) (width 0.25) (layer "B.Cu") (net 3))
 (segment (start 132.195 105.45) (end 131.46 106.185) (width 0.25) (layer "F.Cu") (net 1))
 (segment (start 131.53 106.255) (end 131.46 106.185) (width 0.25) (layer "F.Cu") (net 1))
 (segment (start 131.732901 94.14) (end 132.195 94.602099) (width 0.25) (layer "F.Cu") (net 1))
 (segment (start 131.53 111.64) (end 131.53 106.255) (width 0.25) (layer "F.Cu") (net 1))
 (segment (start 132.195 94.602099) (end 132.195 105.45) (width 0.25) (layer "F.Cu") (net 1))
 (via (at 131.53 111.64) (size 0.8) (drill 0.4) (layers "F.Cu" "B.Cu") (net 1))
 (via (at 131.732901 94.14) (size 0.8) (drill 0.4) (layers "F.Cu" "B.Cu") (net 1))
 (via (at 131.46 106.185) (size 0.8) (drill 0.4) (layers "F.Cu" "B.Cu") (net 1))
 (segment (start 131.582901 93.99) (end 131.732901 94.14) (width 0.25) (layer "B.Cu") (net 1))
 (segment (start 123.72 93.99) (end 131.582901 93.99) (width 0.25) (layer "B.Cu") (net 1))
 (segment (start 123.72 111.77) (end 131.4 111.77) (width 0.25) (layer "B.Cu") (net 1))
 (segment (start 131.4 111.77) (end 131.53 111.64) (width 0.25) (layer "B.Cu") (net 1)))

